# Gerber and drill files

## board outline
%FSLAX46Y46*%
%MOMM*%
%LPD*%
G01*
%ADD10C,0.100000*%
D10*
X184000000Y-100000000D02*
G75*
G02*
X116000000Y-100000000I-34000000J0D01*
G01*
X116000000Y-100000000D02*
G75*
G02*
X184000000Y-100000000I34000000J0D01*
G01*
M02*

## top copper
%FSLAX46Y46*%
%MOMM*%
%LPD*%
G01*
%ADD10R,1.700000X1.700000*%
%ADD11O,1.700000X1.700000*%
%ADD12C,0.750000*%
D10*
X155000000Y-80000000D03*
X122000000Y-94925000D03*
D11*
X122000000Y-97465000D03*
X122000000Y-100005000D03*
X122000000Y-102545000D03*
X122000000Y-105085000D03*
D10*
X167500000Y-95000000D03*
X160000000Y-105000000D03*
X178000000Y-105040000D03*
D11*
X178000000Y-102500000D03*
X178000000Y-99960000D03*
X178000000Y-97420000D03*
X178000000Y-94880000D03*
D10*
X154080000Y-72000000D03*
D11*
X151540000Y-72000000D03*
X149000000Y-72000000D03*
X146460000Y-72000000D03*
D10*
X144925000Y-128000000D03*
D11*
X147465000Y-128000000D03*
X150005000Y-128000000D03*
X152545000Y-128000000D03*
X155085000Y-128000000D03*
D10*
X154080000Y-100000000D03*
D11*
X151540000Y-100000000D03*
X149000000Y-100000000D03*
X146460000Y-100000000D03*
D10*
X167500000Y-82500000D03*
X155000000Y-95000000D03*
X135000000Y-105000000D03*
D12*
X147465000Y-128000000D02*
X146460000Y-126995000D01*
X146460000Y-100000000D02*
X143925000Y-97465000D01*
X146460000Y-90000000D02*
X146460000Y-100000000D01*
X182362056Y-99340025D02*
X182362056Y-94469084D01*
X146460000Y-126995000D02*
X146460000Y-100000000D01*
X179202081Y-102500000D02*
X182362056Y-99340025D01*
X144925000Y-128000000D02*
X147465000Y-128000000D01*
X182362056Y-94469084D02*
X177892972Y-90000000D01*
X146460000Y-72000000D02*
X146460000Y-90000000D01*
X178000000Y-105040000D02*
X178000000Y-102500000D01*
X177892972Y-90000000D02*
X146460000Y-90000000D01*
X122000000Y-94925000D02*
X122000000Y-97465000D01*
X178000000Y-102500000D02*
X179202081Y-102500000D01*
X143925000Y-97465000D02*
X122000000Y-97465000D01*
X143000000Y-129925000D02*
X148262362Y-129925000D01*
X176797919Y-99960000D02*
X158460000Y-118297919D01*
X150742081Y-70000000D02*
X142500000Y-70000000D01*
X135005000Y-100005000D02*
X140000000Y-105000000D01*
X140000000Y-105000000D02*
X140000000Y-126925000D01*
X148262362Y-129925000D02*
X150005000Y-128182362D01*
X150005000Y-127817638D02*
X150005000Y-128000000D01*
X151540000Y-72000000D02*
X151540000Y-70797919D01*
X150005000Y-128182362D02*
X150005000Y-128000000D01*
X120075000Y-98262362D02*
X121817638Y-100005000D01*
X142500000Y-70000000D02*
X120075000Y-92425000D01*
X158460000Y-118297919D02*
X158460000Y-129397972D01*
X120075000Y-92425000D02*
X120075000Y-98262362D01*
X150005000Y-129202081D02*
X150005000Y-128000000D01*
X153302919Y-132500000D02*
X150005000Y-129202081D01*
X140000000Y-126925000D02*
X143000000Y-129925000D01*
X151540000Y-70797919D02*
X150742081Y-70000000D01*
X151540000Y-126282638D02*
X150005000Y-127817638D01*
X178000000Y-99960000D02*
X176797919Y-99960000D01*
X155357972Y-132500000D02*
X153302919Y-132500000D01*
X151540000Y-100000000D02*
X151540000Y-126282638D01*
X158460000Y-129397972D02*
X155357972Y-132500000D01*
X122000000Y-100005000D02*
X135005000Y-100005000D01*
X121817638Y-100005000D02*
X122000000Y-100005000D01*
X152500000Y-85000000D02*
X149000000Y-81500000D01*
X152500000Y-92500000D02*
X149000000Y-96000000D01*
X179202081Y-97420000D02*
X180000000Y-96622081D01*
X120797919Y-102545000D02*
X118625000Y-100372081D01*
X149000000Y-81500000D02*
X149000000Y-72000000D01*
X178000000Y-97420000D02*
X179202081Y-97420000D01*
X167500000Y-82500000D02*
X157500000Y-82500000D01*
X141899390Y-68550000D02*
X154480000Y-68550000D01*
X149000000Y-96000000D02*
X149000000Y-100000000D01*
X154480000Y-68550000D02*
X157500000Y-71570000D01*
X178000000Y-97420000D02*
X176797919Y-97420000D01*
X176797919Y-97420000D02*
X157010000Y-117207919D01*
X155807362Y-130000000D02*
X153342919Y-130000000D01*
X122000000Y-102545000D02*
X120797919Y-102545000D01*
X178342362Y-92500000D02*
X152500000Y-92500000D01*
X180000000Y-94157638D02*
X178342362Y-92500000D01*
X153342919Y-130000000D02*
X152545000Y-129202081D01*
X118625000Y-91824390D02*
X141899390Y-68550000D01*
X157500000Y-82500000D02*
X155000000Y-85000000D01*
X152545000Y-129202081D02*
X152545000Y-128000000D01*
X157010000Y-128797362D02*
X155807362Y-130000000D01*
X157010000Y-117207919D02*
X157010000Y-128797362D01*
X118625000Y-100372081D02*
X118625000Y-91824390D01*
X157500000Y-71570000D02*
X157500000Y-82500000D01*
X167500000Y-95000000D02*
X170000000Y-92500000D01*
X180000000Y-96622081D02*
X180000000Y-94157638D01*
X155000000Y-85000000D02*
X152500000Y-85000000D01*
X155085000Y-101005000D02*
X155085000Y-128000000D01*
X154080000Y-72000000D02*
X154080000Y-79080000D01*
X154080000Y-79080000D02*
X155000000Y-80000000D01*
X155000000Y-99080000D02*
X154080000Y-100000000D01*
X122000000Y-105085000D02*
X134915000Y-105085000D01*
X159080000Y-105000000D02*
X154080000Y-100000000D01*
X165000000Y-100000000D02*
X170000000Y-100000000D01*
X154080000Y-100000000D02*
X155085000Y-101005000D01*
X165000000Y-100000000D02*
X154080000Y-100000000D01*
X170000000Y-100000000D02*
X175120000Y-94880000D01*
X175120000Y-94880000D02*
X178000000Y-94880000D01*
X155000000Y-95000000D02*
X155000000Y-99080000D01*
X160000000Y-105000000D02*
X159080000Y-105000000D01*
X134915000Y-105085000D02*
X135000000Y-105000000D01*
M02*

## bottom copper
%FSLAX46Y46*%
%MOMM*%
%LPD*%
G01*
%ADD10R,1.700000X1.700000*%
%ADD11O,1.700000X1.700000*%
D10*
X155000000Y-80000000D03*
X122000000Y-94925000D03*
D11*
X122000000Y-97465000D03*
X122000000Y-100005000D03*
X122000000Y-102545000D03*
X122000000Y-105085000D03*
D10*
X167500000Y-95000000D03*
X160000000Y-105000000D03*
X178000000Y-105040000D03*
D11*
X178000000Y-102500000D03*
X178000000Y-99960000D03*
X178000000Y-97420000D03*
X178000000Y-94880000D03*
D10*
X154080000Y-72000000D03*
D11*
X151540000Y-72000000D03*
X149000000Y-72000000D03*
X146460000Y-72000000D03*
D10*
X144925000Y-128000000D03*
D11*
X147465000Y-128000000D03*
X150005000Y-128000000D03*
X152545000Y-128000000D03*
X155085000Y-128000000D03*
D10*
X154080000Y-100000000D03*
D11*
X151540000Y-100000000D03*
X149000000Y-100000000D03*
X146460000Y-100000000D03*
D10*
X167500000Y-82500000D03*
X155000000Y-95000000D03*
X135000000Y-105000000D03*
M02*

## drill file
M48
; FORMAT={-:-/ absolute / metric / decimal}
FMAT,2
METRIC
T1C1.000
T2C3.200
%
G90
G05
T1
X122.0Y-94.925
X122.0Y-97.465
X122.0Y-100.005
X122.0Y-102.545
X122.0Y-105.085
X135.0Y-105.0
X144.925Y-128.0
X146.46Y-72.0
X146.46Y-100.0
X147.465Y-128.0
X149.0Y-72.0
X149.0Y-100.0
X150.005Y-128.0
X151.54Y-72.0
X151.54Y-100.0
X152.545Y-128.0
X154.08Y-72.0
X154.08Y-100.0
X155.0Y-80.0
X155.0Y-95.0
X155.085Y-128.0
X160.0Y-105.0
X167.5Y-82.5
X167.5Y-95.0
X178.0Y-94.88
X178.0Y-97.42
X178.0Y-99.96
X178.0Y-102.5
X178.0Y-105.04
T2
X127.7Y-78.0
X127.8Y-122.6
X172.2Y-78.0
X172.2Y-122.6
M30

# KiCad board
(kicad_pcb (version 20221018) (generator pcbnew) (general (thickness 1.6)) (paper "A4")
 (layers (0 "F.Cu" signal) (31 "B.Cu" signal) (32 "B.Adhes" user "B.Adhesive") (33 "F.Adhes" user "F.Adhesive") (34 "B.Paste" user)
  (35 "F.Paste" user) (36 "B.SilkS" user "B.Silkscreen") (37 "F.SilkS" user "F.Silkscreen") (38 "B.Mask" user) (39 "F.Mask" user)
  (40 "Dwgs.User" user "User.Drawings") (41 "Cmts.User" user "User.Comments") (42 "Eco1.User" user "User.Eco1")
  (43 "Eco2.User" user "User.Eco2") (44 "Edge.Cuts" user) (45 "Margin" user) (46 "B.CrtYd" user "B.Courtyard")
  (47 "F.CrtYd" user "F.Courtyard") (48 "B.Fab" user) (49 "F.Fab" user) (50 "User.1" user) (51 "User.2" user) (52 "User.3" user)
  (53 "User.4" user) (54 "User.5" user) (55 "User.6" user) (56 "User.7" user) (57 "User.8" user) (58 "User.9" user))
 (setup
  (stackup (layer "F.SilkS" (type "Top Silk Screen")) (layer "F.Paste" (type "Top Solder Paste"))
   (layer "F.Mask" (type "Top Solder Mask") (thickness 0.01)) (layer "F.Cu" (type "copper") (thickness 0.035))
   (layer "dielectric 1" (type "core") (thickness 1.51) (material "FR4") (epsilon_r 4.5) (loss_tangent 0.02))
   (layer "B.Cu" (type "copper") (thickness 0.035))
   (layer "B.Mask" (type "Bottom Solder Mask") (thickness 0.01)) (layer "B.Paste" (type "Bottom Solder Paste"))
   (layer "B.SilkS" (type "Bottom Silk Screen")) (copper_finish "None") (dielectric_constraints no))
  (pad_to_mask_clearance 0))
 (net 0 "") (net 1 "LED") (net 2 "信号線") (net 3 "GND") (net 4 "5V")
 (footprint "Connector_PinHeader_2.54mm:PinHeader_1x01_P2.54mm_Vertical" (layer "F.Cu") (at 155 80)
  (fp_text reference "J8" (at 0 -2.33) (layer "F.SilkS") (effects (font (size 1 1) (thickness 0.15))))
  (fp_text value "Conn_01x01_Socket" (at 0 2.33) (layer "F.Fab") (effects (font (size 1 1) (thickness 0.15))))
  (pad "1" thru_hole rect (at 0 0) (size 1.7 1.7) (drill 1) (layers "*.Cu" "*.Mask") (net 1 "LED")))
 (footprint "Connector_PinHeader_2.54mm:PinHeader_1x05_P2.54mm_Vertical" (layer "F.Cu") (at 122 94.925)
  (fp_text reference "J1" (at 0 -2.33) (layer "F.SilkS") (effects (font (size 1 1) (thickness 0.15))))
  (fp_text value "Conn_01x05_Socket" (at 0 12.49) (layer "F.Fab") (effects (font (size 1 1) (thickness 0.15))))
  (pad "1" thru_hole rect (at 0 0) (size 1.7 1.7) (drill 1) (layers "*.Cu" "*.Mask") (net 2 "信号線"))
  (pad "2" thru_hole oval (at 0 2.54) (size 1.7 1.7) (drill 1) (layers "*.Cu" "*.Mask") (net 2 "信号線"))
  (pad "3" thru_hole oval (at 0 5.08) (size 1.7 1.7) (drill 1) (layers "*.Cu" "*.Mask") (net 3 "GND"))
  (pad "4" thru_hole oval (at 0 7.62) (size 1.7 1.7) (drill 1) (layers "*.Cu" "*.Mask") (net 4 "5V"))
  (pad "5" thru_hole oval (at 0 10.16) (size 1.7 1.7) (drill 1) (layers "*.Cu" "*.Mask") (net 1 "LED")))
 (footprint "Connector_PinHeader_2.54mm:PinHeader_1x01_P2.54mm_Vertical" (layer "F.Cu") (at 167.5 95)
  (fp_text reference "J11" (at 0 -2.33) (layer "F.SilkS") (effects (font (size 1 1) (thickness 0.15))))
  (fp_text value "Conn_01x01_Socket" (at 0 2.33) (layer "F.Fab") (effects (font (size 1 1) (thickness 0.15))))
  (pad "1" thru_hole rect (at 0 0) (size 1.7 1.7) (drill 1) (layers "*.Cu" "*.Mask") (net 4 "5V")))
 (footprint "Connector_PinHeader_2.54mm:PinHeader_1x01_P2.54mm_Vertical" (layer "F.Cu") (at 160 105)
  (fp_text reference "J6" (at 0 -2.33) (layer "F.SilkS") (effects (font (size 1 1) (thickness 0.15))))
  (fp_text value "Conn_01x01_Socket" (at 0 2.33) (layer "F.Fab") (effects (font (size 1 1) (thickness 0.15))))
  (pad "1" thru_hole rect (at 0 0) (size 1.7 1.7) (drill 1) (layers "*.Cu" "*.Mask") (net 1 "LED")))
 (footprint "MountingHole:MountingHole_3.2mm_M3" (layer "F.Cu") (at 127.8 122.6)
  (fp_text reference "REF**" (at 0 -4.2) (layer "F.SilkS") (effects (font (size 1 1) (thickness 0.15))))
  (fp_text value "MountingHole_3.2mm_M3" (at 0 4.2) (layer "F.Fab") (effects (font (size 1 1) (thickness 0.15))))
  (pad "" np_thru_hole circle (at 0 0) (size 3.2 3.2) (drill 3.2) (layers "*.Cu" "*.Mask")))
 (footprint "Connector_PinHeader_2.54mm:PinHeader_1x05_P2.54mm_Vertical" (layer "F.Cu") (at 178 105.04 180)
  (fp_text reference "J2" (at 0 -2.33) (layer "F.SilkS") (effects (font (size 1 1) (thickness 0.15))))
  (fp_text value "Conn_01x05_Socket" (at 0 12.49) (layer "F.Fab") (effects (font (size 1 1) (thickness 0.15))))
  (pad "1" thru_hole rect (at 0 0 180) (size 1.7 1.7) (drill 1) (layers "*.Cu" "*.Mask") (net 2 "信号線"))
  (pad "2" thru_hole oval (at 0 2.54 180) (size 1.7 1.7) (drill 1) (layers "*.Cu" "*.Mask") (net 2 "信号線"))
  (pad "3" thru_hole oval (at 0 5.08 180) (size 1.7 1.7) (drill 1) (layers "*.Cu" "*.Mask") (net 3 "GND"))
  (pad "4" thru_hole oval (at 0 7.62 180) (size 1.7 1.7) (drill 1) (layers "*.Cu" "*.Mask") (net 4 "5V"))
  (pad "5" thru_hole oval (at 0 10.16 180) (size 1.7 1.7) (drill 1) (layers "*.Cu" "*.Mask") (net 1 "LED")))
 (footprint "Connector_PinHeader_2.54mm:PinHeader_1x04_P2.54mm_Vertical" (layer "F.Cu") (at 154.08 72 -90)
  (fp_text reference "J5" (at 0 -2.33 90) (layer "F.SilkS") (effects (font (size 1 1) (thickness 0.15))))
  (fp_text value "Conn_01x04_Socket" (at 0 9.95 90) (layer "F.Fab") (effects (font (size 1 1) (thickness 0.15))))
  (pad "1" thru_hole rect (at 0 0 270) (size 1.7 1.7) (drill 1) (layers "*.Cu" "*.Mask") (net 1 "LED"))
  (pad "2" thru_hole oval (at 0 2.54 270) (size 1.7 1.7) (drill 1) (layers "*.Cu" "*.Mask") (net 3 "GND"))
  (pad "3" thru_hole oval (at 0 5.08 270) (size 1.7 1.7) (drill 1) (layers "*.Cu" "*.Mask") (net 4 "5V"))
  (pad "4" thru_hole oval (at 0 7.62 270) (size 1.7 1.7) (drill 1) (layers "*.Cu" "*.Mask") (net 2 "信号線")))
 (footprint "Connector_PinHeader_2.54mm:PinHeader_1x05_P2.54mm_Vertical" (layer "F.Cu") (at 144.925 128 90)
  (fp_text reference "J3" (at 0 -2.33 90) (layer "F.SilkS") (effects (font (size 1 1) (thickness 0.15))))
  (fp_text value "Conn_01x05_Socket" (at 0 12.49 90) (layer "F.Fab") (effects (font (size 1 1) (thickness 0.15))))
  (pad "1" thru_hole rect (at 0 0 90) (size 1.7 1.7) (drill 1) (layers "*.Cu" "*.Mask") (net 2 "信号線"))
  (pad "2" thru_hole oval (at 0 2.54 90) (size 1.7 1.7) (drill 1) (layers "*.Cu" "*.Mask") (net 2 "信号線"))
  (pad "3" thru_hole oval (at 0 5.08 90) (size 1.7 1.7) (drill 1) (layers "*.Cu" "*.Mask") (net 3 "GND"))
  (pad "4" thru_hole oval (at 0 7.62 90) (size 1.7 1.7) (drill 1) (layers "*.Cu" "*.Mask") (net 4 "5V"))
  (pad "5" thru_hole oval (at 0 10.16 90) (size 1.7 1.7) (drill 1) (layers "*.Cu" "*.Mask") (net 1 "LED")))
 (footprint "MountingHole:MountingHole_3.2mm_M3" (layer "F.Cu") (at 172.2 122.6)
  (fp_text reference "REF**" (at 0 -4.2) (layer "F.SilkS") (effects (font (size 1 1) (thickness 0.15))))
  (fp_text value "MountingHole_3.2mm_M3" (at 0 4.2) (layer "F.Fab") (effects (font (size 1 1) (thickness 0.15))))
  (pad "" np_thru_hole circle (at 0 0) (size 3.2 3.2) (drill 3.2) (layers "*.Cu" "*.Mask")))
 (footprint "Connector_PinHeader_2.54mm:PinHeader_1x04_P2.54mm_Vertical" (layer "F.Cu") (at 154.08 100 -90)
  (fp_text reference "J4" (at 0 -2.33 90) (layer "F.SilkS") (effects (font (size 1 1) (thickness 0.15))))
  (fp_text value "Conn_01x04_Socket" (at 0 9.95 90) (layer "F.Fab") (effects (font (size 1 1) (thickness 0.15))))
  (pad "1" thru_hole rect (at 0 0 270) (size 1.7 1.7) (drill 1) (layers "*.Cu" "*.Mask") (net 1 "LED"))
  (pad "2" thru_hole oval (at 0 2.54 270) (size 1.7 1.7) (drill 1) (layers "*.Cu" "*.Mask") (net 3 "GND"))
  (pad "3" thru_hole oval (at 0 5.08 270) (size 1.7 1.7) (drill 1) (layers "*.Cu" "*.Mask") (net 4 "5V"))
  (pad "4" thru_hole oval (at 0 7.62 270) (size 1.7 1.7) (drill 1) (layers "*.Cu" "*.Mask") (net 2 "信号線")))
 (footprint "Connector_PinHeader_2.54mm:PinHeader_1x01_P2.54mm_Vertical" (layer "F.Cu") (at 167.5 82.5)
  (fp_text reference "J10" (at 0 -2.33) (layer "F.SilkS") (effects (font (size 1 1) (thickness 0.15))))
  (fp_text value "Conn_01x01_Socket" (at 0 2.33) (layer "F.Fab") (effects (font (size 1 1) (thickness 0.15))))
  (pad "1" thru_hole rect (at 0 0) (size 1.7 1.7) (drill 1) (layers "*.Cu" "*.Mask") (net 4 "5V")))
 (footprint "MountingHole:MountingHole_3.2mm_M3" (layer "F.Cu") (at 172.2 78)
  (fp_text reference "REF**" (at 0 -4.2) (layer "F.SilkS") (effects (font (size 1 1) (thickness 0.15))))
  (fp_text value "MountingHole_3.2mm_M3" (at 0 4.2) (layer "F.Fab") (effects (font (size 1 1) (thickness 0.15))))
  (pad "" np_thru_hole circle (at 0 0) (size 3.2 3.2) (drill 3.2) (layers "*.Cu" "*.Mask")))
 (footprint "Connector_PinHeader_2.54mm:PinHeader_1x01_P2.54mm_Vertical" (layer "F.Cu") (at 155 95)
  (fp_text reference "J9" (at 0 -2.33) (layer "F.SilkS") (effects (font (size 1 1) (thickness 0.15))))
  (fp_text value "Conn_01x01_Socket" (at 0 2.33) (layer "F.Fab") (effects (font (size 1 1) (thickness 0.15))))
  (pad "1" thru_hole rect (at 0 0) (size 1.7 1.7) (drill 1) (layers "*.Cu" "*.Mask") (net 1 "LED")))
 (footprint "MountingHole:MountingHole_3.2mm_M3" (layer "F.Cu") (at 127.7 78)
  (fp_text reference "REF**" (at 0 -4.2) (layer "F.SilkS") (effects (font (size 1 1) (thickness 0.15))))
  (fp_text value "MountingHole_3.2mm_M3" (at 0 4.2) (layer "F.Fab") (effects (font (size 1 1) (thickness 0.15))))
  (pad "" np_thru_hole circle (at 0 0) (size 3.2 3.2) (drill 3.2) (layers "*.Cu" "*.Mask")))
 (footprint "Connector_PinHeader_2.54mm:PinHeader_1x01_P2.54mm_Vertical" (layer "F.Cu") (at 135 105)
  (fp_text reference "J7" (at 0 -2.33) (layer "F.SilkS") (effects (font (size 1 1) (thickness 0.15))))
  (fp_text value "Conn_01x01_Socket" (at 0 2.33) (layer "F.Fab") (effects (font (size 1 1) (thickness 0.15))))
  (pad "1" thru_hole rect (at 0 0) (size 1.7 1.7) (drill 1) (layers "*.Cu" "*.Mask") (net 1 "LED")))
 (gr_circle (center 150 100) (end 184 100) (stroke (width 0.1) (type default)) (fill none) (layer "Edge.Cuts"))
 (segment (start 147.465 128) (end 146.46 126.995) (width 0.75) (layer "F.Cu") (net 2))
 (segment (start 146.46 100) (end 143.925 97.465) (width 0.75) (layer "F.Cu") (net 2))
 (segment (start 146.46 90) (end 146.46 100) (width 0.75) (layer "F.Cu") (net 2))
 (segment (start 182.362056 99.340025) (end 182.362056 94.469084) (width 0.75) (layer "F.Cu") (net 2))
 (segment (start 146.46 126.995) (end 146.46 100) (width 0.75) (layer "F.Cu") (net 2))
 (segment (start 179.202081 102.5) (end 182.362056 99.340025) (width 0.75) (layer "F.Cu") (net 2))
 (segment (start 144.925 128) (end 147.465 128) (width 0.75) (layer "F.Cu") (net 2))
 (segment (start 182.362056 94.469084) (end 177.892972 90) (width 0.75) (layer "F.Cu") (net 2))
 (segment (start 146.46 72) (end 146.46 90) (width 0.75) (layer "F.Cu") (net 2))
 (segment (start 178 105.04) (end 178 102.5) (width 0.75) (layer "F.Cu") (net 2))
 (segment (start 177.892972 90) (end 146.46 90) (width 0.75) (layer "F.Cu") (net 2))
 (segment (start 122 94.925) (end 122 97.465) (width 0.75) (layer "F.Cu") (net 2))
 (segment (start 178 102.5) (end 179.202081 102.5) (width 0.75) (layer "F.Cu") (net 2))
 (segment (start 143.925 97.465) (end 122 97.465) (width 0.75) (layer "F.Cu") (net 2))
 (segment (start 143 129.925) (end 148.262362 129.925) (width 0.75) (layer "F.Cu") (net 3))
 (segment (start 176.797919 99.96) (end 158.46 118.297919) (width 0.75) (layer "F.Cu") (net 3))
 (segment (start 150.742081 70) (end 142.5 70) (width 0.75) (layer "F.Cu") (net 3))
 (segment (start 135.005 100.005) (end 140 105) (width 0.75) (layer "F.Cu") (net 3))
 (segment (start 140 105) (end 140 126.925) (width 0.75) (layer "F.Cu") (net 3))
 (segment (start 148.262362 129.925) (end 150.005 128.182362) (width 0.75) (layer "F.Cu") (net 3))
 (segment (start 150.005 127.817638) (end 150.005 128) (width 0.75) (layer "F.Cu") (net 3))
 (segment (start 151.54 72) (end 151.54 70.797919) (width 0.75) (layer "F.Cu") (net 3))
 (segment (start 150.005 128.182362) (end 150.005 128) (width 0.75) (layer "F.Cu") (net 3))
 (segment (start 120.075 98.262362) (end 121.817638 100.005) (width 0.75) (layer "F.Cu") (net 3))
 (segment (start 142.5 70) (end 120.075 92.425) (width 0.75) (layer "F.Cu") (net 3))
 (segment (start 158.46 118.297919) (end 158.46 129.397972) (width 0.75) (layer "F.Cu") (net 3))
 (segment (start 120.075 92.425) (end 120.075 98.262362) (width 0.75) (layer "F.Cu") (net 3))
 (segment (start 150.005 129.202081) (end 150.005 128) (width 0.75) (layer "F.Cu") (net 3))
 (segment (start 153.302919 132.5) (end 150.005 129.202081) (width 0.75) (layer "F.Cu") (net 3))
 (segment (start 140 126.925) (end 143 129.925) (width 0.75) (layer "F.Cu") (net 3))
 (segment (start 151.54 70.797919) (end 150.742081 70) (width 0.75) (layer "F.Cu") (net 3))
 (segment (start 151.54 126.282638) (end 150.005 127.817638) (width 0.75) (layer "F.Cu") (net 3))
 (segment (start 178 99.96) (end 176.797919 99.96) (width 0.75) (layer "F.Cu") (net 3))
 (segment (start 155.357972 132.5) (end 153.302919 132.5) (width 0.75) (layer "F.Cu") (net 3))
 (segment (start 151.54 100) (end 151.54 126.282638) (width 0.75) (layer "F.Cu") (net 3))
 (segment (start 158.46 129.397972) (end 155.357972 132.5) (width 0.75) (layer "F.Cu") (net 3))
 (segment (start 122 100.005) (end 135.005 100.005) (width 0.75) (layer "F.Cu") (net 3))
 (segment (start 121.817638 100.005) (end 122 100.005) (width 0.75) (layer "F.Cu") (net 3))
 (segment (start 152.5 85) (end 149 81.5) (width 0.75) (layer "F.Cu") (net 4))
 (segment (start 152.5 92.5) (end 149 96) (width 0.75) (layer "F.Cu") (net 4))
 (segment (start 179.202081 97.42) (end 180 96.622081) (width 0.75) (layer "F.Cu") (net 4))
 (segment (start 120.797919 102.545) (end 118.625 100.372081) (width 0.75) (layer "F.Cu") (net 4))
 (segment (start 149 81.5) (end 149 72) (width 0.75) (layer "F.Cu") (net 4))
 (segment (start 178 97.42) (end 179.202081 97.42) (width 0.75) (layer "F.Cu") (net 4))
 (segment (start 167.5 82.5) (end 157.5 82.5) (width 0.75) (layer "F.Cu") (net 4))
 (segment (start 141.89939 68.55) (end 154.48 68.55) (width 0.75) (layer "F.Cu") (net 4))
 (segment (start 149 96) (end 149 100) (width 0.75) (layer "F.Cu") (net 4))
 (segment (start 154.48 68.55) (end 157.5 71.57) (width 0.75) (layer "F.Cu") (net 4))
 (segment (start 178 97.42) (end 176.797919 97.42) (width 0.75) (layer "F.Cu") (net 4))
 (segment (start 176.797919 97.42) (end 157.01 117.207919) (width 0.75) (layer "F.Cu") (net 4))
 (segment (start 155.807362 130) (end 153.342919 130) (width 0.75) (layer "F.Cu") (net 4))
 (segment (start 122 102.545) (end 120.797919 102.545) (width 0.75) (layer "F.Cu") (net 4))
 (segment (start 178.342362 92.5) (end 152.5 92.5) (width 0.75) (layer "F.Cu") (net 4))
 (segment (start 180 94.157638) (end 178.342362 92.5) (width 0.75) (layer "F.Cu") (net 4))
 (segment (start 153.342919 130) (end 152.545 129.202081) (width 0.75) (layer "F.Cu") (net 4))
 (segment (start 118.625 91.82439) (end 141.89939 68.55) (width 0.75) (layer "F.Cu") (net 4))
 (segment (start 157.5 82.5) (end 155 85) (width 0.75) (layer "F.Cu") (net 4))
 (segment (start 152.545 129.202081) (end 152.545 128) (width 0.75) (layer "F.Cu") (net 4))
 (segment (start 157.01 128.797362) (end 155.807362 130) (width 0.75) (layer "F.Cu") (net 4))
 (segment (start 157.01 117.207919) (end 157.01 128.797362) (width 0.75) (layer "F.Cu") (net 4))
 (segment (start 118.625 100.372081) (end 118.625 91.82439) (width 0.75) (layer "F.Cu") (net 4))
 (segment (start 157.5 71.57) (end 157.5 82.5) (width 0.75) (layer "F.Cu") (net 4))
 (segment (start 167.5 95) (end 170 92.5) (width 0.75) (layer "F.Cu") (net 4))
 (segment (start 180 96.622081) (end 180 94.157638) (width 0.75) (layer "F.Cu") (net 4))
 (segment (start 155 85) (end 152.5 85) (width 0.75) (layer "F.Cu") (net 4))
 (segment (start 155.085 101.005) (end 155.085 128) (width 0.75) (layer "F.Cu") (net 1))
 (segment (start 154.08 72) (end 154.08 79.08) (width 0.75) (layer "F.Cu") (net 1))
 (segment (start 154.08 79.08) (end 155 80) (width 0.75) (layer "F.Cu") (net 1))
 (segment (start 155 99.08) (end 154.08 100) (width 0.75) (layer "F.Cu") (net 1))
 (segment (start 122 105.085) (end 134.915 105.085) (width 0.75) (layer "F.Cu") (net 1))
 (segment (start 159.08 105) (end 154.08 100) (width 0.75) (layer "F.Cu") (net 1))
 (segment (start 165 100) (end 170 100) (width 0.75) (layer "F.Cu") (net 1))
 (segment (start 154.08 100) (end 155.085 101.005) (width 0.75) (layer "F.Cu") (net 1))
 (segment (start 165 100) (end 154.08 100) (width 0.75) (layer "F.Cu") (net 1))
 (segment (start 170 100) (end 175.12 94.88) (width 0.75) (layer "F.Cu") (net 1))
 (segment (start 175.12 94.88) (end 178 94.88) (width 0.75) (layer "F.Cu") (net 1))
 (segment (start 155 95) (end 155 99.08) (width 0.75) (layer "F.Cu") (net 1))
 (segment (start 160 105) (end 159.08 105) (width 0.75) (layer "F.Cu") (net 1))
 (segment (start 134.915 105.085) (end 135 105) (width 0.75) (layer "F.Cu") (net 1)))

